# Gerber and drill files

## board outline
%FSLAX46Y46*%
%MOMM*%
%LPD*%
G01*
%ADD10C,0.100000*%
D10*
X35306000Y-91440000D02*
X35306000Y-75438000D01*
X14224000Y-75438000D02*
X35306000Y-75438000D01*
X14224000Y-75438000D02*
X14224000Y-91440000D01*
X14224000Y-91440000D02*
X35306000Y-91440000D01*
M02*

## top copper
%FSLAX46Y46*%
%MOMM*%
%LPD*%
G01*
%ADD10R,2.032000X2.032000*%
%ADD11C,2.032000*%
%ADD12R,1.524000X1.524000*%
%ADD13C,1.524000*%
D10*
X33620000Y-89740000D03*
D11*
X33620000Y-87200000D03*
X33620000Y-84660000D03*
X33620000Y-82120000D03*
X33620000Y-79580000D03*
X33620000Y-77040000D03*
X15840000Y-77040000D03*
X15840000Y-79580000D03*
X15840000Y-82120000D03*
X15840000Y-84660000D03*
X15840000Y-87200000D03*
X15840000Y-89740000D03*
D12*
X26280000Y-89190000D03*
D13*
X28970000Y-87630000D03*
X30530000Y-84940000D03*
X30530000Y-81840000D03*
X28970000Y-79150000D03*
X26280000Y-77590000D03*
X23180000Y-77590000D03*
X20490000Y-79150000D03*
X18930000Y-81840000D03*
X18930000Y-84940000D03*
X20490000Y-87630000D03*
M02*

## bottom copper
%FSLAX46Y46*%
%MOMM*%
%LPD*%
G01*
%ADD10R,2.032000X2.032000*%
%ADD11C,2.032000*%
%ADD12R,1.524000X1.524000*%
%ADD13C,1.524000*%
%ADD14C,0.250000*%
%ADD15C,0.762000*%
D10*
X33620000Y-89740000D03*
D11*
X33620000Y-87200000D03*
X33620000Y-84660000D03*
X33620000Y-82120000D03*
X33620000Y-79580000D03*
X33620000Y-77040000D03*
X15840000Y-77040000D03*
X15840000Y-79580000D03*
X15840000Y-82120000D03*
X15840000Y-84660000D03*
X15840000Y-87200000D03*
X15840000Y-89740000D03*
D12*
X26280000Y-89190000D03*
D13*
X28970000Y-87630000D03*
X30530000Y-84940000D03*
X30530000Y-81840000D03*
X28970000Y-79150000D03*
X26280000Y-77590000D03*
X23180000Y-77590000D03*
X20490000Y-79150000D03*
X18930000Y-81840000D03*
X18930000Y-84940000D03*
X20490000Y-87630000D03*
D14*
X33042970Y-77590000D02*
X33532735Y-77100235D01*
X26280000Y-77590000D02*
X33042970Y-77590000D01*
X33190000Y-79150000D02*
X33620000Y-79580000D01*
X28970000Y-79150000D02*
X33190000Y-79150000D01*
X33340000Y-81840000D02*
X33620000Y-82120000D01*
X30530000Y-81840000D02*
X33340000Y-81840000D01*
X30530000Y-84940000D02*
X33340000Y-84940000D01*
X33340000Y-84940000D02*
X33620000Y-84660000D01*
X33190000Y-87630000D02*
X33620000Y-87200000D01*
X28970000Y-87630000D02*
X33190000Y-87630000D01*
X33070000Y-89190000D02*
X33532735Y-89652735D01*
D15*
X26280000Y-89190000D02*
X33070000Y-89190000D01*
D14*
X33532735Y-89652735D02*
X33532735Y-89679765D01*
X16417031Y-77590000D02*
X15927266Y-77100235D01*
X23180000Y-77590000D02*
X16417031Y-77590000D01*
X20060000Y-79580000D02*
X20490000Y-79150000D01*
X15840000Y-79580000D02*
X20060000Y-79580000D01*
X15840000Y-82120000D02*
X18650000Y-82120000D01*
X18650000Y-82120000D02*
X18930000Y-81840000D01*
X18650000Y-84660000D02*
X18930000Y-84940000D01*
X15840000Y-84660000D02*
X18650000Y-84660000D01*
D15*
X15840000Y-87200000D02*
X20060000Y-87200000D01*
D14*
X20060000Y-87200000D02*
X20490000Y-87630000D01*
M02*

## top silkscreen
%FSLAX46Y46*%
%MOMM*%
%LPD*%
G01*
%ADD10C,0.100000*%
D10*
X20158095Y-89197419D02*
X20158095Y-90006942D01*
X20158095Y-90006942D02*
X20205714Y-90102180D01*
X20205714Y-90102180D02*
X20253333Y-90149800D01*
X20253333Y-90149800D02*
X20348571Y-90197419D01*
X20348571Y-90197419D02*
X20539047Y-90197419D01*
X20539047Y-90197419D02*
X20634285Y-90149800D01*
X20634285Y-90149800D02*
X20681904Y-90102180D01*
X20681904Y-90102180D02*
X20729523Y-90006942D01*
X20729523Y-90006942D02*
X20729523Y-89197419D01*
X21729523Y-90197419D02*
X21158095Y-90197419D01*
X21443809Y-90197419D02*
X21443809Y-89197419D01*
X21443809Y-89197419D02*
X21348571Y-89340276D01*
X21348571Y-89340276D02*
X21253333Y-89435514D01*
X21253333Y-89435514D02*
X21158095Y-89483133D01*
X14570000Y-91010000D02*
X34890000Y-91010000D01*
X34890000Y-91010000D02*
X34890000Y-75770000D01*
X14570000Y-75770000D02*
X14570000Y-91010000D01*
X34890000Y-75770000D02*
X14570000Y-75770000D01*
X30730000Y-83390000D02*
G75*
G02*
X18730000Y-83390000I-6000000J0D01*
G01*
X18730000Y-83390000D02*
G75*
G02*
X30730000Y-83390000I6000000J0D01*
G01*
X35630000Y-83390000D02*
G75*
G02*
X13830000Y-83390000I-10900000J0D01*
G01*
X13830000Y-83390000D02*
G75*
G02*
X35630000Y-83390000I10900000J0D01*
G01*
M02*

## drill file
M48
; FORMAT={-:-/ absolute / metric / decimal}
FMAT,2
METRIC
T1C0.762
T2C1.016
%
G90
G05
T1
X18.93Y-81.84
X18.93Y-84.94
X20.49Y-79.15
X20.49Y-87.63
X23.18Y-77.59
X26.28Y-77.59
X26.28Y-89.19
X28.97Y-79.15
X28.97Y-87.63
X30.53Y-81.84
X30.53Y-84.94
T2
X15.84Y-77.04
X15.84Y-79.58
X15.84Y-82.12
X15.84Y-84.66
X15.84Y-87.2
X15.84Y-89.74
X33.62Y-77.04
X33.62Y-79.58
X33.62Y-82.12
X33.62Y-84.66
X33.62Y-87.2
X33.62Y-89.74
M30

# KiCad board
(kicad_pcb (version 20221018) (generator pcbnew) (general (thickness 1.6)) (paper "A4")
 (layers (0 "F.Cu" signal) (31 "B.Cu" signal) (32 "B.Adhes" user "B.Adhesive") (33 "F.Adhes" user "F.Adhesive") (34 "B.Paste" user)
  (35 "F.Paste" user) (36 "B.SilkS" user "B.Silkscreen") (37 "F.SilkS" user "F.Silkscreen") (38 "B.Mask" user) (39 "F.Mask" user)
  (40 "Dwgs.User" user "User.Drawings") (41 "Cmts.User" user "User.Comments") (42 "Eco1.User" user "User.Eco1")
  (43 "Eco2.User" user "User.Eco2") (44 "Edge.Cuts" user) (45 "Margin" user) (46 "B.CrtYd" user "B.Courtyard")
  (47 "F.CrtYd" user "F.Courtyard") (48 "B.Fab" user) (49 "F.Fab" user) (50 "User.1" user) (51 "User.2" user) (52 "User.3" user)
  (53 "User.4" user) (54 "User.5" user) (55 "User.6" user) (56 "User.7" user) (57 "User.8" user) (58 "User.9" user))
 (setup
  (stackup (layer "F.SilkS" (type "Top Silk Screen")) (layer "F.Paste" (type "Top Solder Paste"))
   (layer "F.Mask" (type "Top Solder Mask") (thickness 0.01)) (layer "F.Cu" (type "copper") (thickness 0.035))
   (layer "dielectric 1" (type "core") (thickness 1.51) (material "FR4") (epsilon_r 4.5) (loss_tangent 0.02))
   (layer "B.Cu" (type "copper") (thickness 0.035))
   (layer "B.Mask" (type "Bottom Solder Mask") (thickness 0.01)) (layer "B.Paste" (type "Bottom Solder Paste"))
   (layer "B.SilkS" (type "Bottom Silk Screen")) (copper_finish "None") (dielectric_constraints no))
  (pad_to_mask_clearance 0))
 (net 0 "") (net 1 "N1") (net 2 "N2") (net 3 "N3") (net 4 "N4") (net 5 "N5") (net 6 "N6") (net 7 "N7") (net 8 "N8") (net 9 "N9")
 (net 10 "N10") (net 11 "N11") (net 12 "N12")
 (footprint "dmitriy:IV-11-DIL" (layer "F.Cu") (at 24.73 83.39 90)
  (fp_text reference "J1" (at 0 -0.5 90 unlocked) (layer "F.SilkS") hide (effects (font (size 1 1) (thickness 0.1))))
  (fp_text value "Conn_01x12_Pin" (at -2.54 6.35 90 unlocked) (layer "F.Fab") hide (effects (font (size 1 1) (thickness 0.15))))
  (fp_line (start -7.62 -10.16) (end -7.62 10.16) (stroke (width 0.1) (type default)) (layer "F.SilkS"))
  (fp_line (start -7.62 10.16) (end 7.62 10.16) (stroke (width 0.1) (type default)) (layer "F.SilkS"))
  (fp_line (start 7.62 -10.16) (end -7.62 -10.16) (stroke (width 0.1) (type default)) (layer "F.SilkS"))
  (fp_line (start 7.62 10.16) (end 7.62 -10.16) (stroke (width 0.1) (type default)) (layer "F.SilkS"))
  (pad "1" thru_hole rect (at -6.35 8.89 90) (size 2.032 2.032) (drill 1.016) (layers "*.Cu" "*.Mask") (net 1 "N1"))
  (pad "2" thru_hole circle (at -3.81 8.89 90) (size 2.032 2.032) (drill 1.016) (layers "*.Cu" "*.Mask") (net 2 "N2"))
  (pad "3" thru_hole circle (at -1.27 8.89 90) (size 2.032 2.032) (drill 1.016) (layers "*.Cu" "*.Mask") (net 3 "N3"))
  (pad "4" thru_hole circle (at 1.27 8.89 90) (size 2.032 2.032) (drill 1.016) (layers "*.Cu" "*.Mask") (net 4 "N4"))
  (pad "5" thru_hole circle (at 3.81 8.89 90) (size 2.032 2.032) (drill 1.016) (layers "*.Cu" "*.Mask") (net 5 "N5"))
  (pad "6" thru_hole circle (at 6.35 8.89 90) (size 2.032 2.032) (drill 1.016) (layers "*.Cu" "*.Mask") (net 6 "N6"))
  (pad "7" thru_hole circle (at 6.35 -8.89 90) (size 2.032 2.032) (drill 1.016) (layers "*.Cu" "*.Mask") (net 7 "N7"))
  (pad "8" thru_hole circle (at 3.81 -8.89 90) (size 2.032 2.032) (drill 1.016) (layers "*.Cu" "*.Mask") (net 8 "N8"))
  (pad "9" thru_hole circle (at 1.27 -8.89 90) (size 2.032 2.032) (drill 1.016) (layers "*.Cu" "*.Mask") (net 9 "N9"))
  (pad "10" thru_hole circle (at -1.27 -8.89 90) (size 2.032 2.032) (drill 1.016) (layers "*.Cu" "*.Mask") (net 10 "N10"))
  (pad "11" thru_hole circle (at -3.81 -8.89 90) (size 2.032 2.032) (drill 1.016) (layers "*.Cu" "*.Mask") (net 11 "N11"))
  (pad "12" thru_hole circle (at -6.35 -8.89 90) (size 2.032 2.032) (drill 1.016) (layers "*.Cu" "*.Mask") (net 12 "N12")))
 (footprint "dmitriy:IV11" (layer "F.Cu") (at 24.73 83.39)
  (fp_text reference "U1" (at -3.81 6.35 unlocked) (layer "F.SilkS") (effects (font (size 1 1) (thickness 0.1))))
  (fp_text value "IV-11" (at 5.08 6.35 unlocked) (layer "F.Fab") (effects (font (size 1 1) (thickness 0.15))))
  (fp_circle (center 0 0) (end 6 0) (stroke (width 0.1) (type default)) (fill none) (layer "F.SilkS"))
  (fp_circle (center 0 0) (end 10.9 0) (stroke (width 0.1) (type default)) (fill none) (layer "F.SilkS"))
  (pad "1" thru_hole rect (at 1.55 5.8) (size 1.524 1.524) (drill 0.762) (layers "*.Cu" "*.Mask") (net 1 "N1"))
  (pad "2" thru_hole circle (at 4.24 4.24) (size 1.524 1.524) (drill 0.762) (layers "*.Cu" "*.Mask") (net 2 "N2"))
  (pad "3" thru_hole circle (at 5.8 1.55) (size 1.524 1.524) (drill 0.762) (layers "*.Cu" "*.Mask") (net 3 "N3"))
  (pad "4" thru_hole circle (at 5.8 -1.55) (size 1.524 1.524) (drill 0.762) (layers "*.Cu" "*.Mask") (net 4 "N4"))
  (pad "5" thru_hole circle (at 4.24 -4.24) (size 1.524 1.524) (drill 0.762) (layers "*.Cu" "*.Mask") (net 5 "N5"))
  (pad "6" thru_hole circle (at 1.55 -5.8) (size 1.524 1.524) (drill 0.762) (layers "*.Cu" "*.Mask") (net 6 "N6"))
  (pad "7" thru_hole circle (at -1.55 -5.8) (size 1.524 1.524) (drill 0.762) (layers "*.Cu" "*.Mask") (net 7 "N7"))
  (pad "8" thru_hole circle (at -4.24 -4.24) (size 1.524 1.524) (drill 0.762) (layers "*.Cu" "*.Mask") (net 8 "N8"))
  (pad "9" thru_hole circle (at -5.8 -1.55) (size 1.524 1.524) (drill 0.762) (layers "*.Cu" "*.Mask") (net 9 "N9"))
  (pad "10" thru_hole circle (at -5.8 1.55) (size 1.524 1.524) (drill 0.762) (layers "*.Cu" "*.Mask") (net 10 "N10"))
  (pad "11" thru_hole circle (at -4.24 4.24) (size 1.524 1.524) (drill 0.762) (layers "*.Cu" "*.Mask") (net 11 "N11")))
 (gr_line (start 35.306 91.44) (end 35.306 75.438) (stroke (width 0.1) (type default)) (layer "Edge.Cuts"))
 (gr_line (start 14.224 75.438) (end 35.306 75.438) (stroke (width 0.1) (type default)) (layer "Edge.Cuts"))
 (gr_line (start 14.224 75.438) (end 14.224 91.44) (stroke (width 0.1) (type default)) (layer "Edge.Cuts"))
 (gr_line (start 14.224 91.44) (end 35.306 91.44) (stroke (width 0.1) (type default)) (layer "Edge.Cuts"))
 (segment (start 33.04297 77.59) (end 33.532735 77.100235) (width 0.25) (layer "B.Cu") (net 6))
 (segment (start 26.28 77.59) (end 33.04297 77.59) (width 0.25) (layer "B.Cu") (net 6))
 (segment (start 33.19 79.15) (end 33.62 79.58) (width 0.25) (layer "B.Cu") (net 5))
 (segment (start 28.97 79.15) (end 33.19 79.15) (width 0.25) (layer "B.Cu") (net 5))
 (segment (start 33.34 81.84) (end 33.62 82.12) (width 0.25) (layer "B.Cu") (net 4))
 (segment (start 30.53 81.84) (end 33.34 81.84) (width 0.25) (layer "B.Cu") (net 4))
 (segment (start 30.53 84.94) (end 33.34 84.94) (width 0.25) (layer "B.Cu") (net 3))
 (segment (start 33.34 84.94) (end 33.62 84.66) (width 0.25) (layer "B.Cu") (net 3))
 (segment (start 33.19 87.63) (end 33.62 87.2) (width 0.25) (layer "B.Cu") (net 2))
 (segment (start 28.97 87.63) (end 33.19 87.63) (width 0.25) (layer "B.Cu") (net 2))
 (segment (start 33.07 89.19) (end 33.532735 89.652735) (width 0.25) (layer "B.Cu") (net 1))
 (segment (start 26.28 89.19) (end 33.07 89.19) (width 0.762) (layer "B.Cu") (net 1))
 (segment (start 33.532735 89.652735) (end 33.532735 89.679765) (width 0.25) (layer "B.Cu") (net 1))
 (segment (start 16.417031 77.59) (end 15.927266 77.100235) (width 0.25) (layer "B.Cu") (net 7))
 (segment (start 23.18 77.59) (end 16.417031 77.59) (width 0.25) (layer "B.Cu") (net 7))
 (segment (start 20.06 79.58) (end 20.49 79.15) (width 0.25) (layer "B.Cu") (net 8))
 (segment (start 15.84 79.58) (end 20.06 79.58) (width 0.25) (layer "B.Cu") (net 8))
 (segment (start 15.84 82.12) (end 18.65 82.12) (width 0.25) (layer "B.Cu") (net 9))
 (segment (start 18.65 82.12) (end 18.93 81.84) (width 0.25) (layer "B.Cu") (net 9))
 (segment (start 18.65 84.66) (end 18.93 84.94) (width 0.25) (layer "B.Cu") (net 10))
 (segment (start 15.84 84.66) (end 18.65 84.66) (width 0.25) (layer "B.Cu") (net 10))
 (segment (start 15.84 87.2) (end 20.06 87.2) (width 0.762) (layer "B.Cu") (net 11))
 (segment (start 20.06 87.2) (end 20.49 87.63) (width 0.25) (layer "B.Cu") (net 11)))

